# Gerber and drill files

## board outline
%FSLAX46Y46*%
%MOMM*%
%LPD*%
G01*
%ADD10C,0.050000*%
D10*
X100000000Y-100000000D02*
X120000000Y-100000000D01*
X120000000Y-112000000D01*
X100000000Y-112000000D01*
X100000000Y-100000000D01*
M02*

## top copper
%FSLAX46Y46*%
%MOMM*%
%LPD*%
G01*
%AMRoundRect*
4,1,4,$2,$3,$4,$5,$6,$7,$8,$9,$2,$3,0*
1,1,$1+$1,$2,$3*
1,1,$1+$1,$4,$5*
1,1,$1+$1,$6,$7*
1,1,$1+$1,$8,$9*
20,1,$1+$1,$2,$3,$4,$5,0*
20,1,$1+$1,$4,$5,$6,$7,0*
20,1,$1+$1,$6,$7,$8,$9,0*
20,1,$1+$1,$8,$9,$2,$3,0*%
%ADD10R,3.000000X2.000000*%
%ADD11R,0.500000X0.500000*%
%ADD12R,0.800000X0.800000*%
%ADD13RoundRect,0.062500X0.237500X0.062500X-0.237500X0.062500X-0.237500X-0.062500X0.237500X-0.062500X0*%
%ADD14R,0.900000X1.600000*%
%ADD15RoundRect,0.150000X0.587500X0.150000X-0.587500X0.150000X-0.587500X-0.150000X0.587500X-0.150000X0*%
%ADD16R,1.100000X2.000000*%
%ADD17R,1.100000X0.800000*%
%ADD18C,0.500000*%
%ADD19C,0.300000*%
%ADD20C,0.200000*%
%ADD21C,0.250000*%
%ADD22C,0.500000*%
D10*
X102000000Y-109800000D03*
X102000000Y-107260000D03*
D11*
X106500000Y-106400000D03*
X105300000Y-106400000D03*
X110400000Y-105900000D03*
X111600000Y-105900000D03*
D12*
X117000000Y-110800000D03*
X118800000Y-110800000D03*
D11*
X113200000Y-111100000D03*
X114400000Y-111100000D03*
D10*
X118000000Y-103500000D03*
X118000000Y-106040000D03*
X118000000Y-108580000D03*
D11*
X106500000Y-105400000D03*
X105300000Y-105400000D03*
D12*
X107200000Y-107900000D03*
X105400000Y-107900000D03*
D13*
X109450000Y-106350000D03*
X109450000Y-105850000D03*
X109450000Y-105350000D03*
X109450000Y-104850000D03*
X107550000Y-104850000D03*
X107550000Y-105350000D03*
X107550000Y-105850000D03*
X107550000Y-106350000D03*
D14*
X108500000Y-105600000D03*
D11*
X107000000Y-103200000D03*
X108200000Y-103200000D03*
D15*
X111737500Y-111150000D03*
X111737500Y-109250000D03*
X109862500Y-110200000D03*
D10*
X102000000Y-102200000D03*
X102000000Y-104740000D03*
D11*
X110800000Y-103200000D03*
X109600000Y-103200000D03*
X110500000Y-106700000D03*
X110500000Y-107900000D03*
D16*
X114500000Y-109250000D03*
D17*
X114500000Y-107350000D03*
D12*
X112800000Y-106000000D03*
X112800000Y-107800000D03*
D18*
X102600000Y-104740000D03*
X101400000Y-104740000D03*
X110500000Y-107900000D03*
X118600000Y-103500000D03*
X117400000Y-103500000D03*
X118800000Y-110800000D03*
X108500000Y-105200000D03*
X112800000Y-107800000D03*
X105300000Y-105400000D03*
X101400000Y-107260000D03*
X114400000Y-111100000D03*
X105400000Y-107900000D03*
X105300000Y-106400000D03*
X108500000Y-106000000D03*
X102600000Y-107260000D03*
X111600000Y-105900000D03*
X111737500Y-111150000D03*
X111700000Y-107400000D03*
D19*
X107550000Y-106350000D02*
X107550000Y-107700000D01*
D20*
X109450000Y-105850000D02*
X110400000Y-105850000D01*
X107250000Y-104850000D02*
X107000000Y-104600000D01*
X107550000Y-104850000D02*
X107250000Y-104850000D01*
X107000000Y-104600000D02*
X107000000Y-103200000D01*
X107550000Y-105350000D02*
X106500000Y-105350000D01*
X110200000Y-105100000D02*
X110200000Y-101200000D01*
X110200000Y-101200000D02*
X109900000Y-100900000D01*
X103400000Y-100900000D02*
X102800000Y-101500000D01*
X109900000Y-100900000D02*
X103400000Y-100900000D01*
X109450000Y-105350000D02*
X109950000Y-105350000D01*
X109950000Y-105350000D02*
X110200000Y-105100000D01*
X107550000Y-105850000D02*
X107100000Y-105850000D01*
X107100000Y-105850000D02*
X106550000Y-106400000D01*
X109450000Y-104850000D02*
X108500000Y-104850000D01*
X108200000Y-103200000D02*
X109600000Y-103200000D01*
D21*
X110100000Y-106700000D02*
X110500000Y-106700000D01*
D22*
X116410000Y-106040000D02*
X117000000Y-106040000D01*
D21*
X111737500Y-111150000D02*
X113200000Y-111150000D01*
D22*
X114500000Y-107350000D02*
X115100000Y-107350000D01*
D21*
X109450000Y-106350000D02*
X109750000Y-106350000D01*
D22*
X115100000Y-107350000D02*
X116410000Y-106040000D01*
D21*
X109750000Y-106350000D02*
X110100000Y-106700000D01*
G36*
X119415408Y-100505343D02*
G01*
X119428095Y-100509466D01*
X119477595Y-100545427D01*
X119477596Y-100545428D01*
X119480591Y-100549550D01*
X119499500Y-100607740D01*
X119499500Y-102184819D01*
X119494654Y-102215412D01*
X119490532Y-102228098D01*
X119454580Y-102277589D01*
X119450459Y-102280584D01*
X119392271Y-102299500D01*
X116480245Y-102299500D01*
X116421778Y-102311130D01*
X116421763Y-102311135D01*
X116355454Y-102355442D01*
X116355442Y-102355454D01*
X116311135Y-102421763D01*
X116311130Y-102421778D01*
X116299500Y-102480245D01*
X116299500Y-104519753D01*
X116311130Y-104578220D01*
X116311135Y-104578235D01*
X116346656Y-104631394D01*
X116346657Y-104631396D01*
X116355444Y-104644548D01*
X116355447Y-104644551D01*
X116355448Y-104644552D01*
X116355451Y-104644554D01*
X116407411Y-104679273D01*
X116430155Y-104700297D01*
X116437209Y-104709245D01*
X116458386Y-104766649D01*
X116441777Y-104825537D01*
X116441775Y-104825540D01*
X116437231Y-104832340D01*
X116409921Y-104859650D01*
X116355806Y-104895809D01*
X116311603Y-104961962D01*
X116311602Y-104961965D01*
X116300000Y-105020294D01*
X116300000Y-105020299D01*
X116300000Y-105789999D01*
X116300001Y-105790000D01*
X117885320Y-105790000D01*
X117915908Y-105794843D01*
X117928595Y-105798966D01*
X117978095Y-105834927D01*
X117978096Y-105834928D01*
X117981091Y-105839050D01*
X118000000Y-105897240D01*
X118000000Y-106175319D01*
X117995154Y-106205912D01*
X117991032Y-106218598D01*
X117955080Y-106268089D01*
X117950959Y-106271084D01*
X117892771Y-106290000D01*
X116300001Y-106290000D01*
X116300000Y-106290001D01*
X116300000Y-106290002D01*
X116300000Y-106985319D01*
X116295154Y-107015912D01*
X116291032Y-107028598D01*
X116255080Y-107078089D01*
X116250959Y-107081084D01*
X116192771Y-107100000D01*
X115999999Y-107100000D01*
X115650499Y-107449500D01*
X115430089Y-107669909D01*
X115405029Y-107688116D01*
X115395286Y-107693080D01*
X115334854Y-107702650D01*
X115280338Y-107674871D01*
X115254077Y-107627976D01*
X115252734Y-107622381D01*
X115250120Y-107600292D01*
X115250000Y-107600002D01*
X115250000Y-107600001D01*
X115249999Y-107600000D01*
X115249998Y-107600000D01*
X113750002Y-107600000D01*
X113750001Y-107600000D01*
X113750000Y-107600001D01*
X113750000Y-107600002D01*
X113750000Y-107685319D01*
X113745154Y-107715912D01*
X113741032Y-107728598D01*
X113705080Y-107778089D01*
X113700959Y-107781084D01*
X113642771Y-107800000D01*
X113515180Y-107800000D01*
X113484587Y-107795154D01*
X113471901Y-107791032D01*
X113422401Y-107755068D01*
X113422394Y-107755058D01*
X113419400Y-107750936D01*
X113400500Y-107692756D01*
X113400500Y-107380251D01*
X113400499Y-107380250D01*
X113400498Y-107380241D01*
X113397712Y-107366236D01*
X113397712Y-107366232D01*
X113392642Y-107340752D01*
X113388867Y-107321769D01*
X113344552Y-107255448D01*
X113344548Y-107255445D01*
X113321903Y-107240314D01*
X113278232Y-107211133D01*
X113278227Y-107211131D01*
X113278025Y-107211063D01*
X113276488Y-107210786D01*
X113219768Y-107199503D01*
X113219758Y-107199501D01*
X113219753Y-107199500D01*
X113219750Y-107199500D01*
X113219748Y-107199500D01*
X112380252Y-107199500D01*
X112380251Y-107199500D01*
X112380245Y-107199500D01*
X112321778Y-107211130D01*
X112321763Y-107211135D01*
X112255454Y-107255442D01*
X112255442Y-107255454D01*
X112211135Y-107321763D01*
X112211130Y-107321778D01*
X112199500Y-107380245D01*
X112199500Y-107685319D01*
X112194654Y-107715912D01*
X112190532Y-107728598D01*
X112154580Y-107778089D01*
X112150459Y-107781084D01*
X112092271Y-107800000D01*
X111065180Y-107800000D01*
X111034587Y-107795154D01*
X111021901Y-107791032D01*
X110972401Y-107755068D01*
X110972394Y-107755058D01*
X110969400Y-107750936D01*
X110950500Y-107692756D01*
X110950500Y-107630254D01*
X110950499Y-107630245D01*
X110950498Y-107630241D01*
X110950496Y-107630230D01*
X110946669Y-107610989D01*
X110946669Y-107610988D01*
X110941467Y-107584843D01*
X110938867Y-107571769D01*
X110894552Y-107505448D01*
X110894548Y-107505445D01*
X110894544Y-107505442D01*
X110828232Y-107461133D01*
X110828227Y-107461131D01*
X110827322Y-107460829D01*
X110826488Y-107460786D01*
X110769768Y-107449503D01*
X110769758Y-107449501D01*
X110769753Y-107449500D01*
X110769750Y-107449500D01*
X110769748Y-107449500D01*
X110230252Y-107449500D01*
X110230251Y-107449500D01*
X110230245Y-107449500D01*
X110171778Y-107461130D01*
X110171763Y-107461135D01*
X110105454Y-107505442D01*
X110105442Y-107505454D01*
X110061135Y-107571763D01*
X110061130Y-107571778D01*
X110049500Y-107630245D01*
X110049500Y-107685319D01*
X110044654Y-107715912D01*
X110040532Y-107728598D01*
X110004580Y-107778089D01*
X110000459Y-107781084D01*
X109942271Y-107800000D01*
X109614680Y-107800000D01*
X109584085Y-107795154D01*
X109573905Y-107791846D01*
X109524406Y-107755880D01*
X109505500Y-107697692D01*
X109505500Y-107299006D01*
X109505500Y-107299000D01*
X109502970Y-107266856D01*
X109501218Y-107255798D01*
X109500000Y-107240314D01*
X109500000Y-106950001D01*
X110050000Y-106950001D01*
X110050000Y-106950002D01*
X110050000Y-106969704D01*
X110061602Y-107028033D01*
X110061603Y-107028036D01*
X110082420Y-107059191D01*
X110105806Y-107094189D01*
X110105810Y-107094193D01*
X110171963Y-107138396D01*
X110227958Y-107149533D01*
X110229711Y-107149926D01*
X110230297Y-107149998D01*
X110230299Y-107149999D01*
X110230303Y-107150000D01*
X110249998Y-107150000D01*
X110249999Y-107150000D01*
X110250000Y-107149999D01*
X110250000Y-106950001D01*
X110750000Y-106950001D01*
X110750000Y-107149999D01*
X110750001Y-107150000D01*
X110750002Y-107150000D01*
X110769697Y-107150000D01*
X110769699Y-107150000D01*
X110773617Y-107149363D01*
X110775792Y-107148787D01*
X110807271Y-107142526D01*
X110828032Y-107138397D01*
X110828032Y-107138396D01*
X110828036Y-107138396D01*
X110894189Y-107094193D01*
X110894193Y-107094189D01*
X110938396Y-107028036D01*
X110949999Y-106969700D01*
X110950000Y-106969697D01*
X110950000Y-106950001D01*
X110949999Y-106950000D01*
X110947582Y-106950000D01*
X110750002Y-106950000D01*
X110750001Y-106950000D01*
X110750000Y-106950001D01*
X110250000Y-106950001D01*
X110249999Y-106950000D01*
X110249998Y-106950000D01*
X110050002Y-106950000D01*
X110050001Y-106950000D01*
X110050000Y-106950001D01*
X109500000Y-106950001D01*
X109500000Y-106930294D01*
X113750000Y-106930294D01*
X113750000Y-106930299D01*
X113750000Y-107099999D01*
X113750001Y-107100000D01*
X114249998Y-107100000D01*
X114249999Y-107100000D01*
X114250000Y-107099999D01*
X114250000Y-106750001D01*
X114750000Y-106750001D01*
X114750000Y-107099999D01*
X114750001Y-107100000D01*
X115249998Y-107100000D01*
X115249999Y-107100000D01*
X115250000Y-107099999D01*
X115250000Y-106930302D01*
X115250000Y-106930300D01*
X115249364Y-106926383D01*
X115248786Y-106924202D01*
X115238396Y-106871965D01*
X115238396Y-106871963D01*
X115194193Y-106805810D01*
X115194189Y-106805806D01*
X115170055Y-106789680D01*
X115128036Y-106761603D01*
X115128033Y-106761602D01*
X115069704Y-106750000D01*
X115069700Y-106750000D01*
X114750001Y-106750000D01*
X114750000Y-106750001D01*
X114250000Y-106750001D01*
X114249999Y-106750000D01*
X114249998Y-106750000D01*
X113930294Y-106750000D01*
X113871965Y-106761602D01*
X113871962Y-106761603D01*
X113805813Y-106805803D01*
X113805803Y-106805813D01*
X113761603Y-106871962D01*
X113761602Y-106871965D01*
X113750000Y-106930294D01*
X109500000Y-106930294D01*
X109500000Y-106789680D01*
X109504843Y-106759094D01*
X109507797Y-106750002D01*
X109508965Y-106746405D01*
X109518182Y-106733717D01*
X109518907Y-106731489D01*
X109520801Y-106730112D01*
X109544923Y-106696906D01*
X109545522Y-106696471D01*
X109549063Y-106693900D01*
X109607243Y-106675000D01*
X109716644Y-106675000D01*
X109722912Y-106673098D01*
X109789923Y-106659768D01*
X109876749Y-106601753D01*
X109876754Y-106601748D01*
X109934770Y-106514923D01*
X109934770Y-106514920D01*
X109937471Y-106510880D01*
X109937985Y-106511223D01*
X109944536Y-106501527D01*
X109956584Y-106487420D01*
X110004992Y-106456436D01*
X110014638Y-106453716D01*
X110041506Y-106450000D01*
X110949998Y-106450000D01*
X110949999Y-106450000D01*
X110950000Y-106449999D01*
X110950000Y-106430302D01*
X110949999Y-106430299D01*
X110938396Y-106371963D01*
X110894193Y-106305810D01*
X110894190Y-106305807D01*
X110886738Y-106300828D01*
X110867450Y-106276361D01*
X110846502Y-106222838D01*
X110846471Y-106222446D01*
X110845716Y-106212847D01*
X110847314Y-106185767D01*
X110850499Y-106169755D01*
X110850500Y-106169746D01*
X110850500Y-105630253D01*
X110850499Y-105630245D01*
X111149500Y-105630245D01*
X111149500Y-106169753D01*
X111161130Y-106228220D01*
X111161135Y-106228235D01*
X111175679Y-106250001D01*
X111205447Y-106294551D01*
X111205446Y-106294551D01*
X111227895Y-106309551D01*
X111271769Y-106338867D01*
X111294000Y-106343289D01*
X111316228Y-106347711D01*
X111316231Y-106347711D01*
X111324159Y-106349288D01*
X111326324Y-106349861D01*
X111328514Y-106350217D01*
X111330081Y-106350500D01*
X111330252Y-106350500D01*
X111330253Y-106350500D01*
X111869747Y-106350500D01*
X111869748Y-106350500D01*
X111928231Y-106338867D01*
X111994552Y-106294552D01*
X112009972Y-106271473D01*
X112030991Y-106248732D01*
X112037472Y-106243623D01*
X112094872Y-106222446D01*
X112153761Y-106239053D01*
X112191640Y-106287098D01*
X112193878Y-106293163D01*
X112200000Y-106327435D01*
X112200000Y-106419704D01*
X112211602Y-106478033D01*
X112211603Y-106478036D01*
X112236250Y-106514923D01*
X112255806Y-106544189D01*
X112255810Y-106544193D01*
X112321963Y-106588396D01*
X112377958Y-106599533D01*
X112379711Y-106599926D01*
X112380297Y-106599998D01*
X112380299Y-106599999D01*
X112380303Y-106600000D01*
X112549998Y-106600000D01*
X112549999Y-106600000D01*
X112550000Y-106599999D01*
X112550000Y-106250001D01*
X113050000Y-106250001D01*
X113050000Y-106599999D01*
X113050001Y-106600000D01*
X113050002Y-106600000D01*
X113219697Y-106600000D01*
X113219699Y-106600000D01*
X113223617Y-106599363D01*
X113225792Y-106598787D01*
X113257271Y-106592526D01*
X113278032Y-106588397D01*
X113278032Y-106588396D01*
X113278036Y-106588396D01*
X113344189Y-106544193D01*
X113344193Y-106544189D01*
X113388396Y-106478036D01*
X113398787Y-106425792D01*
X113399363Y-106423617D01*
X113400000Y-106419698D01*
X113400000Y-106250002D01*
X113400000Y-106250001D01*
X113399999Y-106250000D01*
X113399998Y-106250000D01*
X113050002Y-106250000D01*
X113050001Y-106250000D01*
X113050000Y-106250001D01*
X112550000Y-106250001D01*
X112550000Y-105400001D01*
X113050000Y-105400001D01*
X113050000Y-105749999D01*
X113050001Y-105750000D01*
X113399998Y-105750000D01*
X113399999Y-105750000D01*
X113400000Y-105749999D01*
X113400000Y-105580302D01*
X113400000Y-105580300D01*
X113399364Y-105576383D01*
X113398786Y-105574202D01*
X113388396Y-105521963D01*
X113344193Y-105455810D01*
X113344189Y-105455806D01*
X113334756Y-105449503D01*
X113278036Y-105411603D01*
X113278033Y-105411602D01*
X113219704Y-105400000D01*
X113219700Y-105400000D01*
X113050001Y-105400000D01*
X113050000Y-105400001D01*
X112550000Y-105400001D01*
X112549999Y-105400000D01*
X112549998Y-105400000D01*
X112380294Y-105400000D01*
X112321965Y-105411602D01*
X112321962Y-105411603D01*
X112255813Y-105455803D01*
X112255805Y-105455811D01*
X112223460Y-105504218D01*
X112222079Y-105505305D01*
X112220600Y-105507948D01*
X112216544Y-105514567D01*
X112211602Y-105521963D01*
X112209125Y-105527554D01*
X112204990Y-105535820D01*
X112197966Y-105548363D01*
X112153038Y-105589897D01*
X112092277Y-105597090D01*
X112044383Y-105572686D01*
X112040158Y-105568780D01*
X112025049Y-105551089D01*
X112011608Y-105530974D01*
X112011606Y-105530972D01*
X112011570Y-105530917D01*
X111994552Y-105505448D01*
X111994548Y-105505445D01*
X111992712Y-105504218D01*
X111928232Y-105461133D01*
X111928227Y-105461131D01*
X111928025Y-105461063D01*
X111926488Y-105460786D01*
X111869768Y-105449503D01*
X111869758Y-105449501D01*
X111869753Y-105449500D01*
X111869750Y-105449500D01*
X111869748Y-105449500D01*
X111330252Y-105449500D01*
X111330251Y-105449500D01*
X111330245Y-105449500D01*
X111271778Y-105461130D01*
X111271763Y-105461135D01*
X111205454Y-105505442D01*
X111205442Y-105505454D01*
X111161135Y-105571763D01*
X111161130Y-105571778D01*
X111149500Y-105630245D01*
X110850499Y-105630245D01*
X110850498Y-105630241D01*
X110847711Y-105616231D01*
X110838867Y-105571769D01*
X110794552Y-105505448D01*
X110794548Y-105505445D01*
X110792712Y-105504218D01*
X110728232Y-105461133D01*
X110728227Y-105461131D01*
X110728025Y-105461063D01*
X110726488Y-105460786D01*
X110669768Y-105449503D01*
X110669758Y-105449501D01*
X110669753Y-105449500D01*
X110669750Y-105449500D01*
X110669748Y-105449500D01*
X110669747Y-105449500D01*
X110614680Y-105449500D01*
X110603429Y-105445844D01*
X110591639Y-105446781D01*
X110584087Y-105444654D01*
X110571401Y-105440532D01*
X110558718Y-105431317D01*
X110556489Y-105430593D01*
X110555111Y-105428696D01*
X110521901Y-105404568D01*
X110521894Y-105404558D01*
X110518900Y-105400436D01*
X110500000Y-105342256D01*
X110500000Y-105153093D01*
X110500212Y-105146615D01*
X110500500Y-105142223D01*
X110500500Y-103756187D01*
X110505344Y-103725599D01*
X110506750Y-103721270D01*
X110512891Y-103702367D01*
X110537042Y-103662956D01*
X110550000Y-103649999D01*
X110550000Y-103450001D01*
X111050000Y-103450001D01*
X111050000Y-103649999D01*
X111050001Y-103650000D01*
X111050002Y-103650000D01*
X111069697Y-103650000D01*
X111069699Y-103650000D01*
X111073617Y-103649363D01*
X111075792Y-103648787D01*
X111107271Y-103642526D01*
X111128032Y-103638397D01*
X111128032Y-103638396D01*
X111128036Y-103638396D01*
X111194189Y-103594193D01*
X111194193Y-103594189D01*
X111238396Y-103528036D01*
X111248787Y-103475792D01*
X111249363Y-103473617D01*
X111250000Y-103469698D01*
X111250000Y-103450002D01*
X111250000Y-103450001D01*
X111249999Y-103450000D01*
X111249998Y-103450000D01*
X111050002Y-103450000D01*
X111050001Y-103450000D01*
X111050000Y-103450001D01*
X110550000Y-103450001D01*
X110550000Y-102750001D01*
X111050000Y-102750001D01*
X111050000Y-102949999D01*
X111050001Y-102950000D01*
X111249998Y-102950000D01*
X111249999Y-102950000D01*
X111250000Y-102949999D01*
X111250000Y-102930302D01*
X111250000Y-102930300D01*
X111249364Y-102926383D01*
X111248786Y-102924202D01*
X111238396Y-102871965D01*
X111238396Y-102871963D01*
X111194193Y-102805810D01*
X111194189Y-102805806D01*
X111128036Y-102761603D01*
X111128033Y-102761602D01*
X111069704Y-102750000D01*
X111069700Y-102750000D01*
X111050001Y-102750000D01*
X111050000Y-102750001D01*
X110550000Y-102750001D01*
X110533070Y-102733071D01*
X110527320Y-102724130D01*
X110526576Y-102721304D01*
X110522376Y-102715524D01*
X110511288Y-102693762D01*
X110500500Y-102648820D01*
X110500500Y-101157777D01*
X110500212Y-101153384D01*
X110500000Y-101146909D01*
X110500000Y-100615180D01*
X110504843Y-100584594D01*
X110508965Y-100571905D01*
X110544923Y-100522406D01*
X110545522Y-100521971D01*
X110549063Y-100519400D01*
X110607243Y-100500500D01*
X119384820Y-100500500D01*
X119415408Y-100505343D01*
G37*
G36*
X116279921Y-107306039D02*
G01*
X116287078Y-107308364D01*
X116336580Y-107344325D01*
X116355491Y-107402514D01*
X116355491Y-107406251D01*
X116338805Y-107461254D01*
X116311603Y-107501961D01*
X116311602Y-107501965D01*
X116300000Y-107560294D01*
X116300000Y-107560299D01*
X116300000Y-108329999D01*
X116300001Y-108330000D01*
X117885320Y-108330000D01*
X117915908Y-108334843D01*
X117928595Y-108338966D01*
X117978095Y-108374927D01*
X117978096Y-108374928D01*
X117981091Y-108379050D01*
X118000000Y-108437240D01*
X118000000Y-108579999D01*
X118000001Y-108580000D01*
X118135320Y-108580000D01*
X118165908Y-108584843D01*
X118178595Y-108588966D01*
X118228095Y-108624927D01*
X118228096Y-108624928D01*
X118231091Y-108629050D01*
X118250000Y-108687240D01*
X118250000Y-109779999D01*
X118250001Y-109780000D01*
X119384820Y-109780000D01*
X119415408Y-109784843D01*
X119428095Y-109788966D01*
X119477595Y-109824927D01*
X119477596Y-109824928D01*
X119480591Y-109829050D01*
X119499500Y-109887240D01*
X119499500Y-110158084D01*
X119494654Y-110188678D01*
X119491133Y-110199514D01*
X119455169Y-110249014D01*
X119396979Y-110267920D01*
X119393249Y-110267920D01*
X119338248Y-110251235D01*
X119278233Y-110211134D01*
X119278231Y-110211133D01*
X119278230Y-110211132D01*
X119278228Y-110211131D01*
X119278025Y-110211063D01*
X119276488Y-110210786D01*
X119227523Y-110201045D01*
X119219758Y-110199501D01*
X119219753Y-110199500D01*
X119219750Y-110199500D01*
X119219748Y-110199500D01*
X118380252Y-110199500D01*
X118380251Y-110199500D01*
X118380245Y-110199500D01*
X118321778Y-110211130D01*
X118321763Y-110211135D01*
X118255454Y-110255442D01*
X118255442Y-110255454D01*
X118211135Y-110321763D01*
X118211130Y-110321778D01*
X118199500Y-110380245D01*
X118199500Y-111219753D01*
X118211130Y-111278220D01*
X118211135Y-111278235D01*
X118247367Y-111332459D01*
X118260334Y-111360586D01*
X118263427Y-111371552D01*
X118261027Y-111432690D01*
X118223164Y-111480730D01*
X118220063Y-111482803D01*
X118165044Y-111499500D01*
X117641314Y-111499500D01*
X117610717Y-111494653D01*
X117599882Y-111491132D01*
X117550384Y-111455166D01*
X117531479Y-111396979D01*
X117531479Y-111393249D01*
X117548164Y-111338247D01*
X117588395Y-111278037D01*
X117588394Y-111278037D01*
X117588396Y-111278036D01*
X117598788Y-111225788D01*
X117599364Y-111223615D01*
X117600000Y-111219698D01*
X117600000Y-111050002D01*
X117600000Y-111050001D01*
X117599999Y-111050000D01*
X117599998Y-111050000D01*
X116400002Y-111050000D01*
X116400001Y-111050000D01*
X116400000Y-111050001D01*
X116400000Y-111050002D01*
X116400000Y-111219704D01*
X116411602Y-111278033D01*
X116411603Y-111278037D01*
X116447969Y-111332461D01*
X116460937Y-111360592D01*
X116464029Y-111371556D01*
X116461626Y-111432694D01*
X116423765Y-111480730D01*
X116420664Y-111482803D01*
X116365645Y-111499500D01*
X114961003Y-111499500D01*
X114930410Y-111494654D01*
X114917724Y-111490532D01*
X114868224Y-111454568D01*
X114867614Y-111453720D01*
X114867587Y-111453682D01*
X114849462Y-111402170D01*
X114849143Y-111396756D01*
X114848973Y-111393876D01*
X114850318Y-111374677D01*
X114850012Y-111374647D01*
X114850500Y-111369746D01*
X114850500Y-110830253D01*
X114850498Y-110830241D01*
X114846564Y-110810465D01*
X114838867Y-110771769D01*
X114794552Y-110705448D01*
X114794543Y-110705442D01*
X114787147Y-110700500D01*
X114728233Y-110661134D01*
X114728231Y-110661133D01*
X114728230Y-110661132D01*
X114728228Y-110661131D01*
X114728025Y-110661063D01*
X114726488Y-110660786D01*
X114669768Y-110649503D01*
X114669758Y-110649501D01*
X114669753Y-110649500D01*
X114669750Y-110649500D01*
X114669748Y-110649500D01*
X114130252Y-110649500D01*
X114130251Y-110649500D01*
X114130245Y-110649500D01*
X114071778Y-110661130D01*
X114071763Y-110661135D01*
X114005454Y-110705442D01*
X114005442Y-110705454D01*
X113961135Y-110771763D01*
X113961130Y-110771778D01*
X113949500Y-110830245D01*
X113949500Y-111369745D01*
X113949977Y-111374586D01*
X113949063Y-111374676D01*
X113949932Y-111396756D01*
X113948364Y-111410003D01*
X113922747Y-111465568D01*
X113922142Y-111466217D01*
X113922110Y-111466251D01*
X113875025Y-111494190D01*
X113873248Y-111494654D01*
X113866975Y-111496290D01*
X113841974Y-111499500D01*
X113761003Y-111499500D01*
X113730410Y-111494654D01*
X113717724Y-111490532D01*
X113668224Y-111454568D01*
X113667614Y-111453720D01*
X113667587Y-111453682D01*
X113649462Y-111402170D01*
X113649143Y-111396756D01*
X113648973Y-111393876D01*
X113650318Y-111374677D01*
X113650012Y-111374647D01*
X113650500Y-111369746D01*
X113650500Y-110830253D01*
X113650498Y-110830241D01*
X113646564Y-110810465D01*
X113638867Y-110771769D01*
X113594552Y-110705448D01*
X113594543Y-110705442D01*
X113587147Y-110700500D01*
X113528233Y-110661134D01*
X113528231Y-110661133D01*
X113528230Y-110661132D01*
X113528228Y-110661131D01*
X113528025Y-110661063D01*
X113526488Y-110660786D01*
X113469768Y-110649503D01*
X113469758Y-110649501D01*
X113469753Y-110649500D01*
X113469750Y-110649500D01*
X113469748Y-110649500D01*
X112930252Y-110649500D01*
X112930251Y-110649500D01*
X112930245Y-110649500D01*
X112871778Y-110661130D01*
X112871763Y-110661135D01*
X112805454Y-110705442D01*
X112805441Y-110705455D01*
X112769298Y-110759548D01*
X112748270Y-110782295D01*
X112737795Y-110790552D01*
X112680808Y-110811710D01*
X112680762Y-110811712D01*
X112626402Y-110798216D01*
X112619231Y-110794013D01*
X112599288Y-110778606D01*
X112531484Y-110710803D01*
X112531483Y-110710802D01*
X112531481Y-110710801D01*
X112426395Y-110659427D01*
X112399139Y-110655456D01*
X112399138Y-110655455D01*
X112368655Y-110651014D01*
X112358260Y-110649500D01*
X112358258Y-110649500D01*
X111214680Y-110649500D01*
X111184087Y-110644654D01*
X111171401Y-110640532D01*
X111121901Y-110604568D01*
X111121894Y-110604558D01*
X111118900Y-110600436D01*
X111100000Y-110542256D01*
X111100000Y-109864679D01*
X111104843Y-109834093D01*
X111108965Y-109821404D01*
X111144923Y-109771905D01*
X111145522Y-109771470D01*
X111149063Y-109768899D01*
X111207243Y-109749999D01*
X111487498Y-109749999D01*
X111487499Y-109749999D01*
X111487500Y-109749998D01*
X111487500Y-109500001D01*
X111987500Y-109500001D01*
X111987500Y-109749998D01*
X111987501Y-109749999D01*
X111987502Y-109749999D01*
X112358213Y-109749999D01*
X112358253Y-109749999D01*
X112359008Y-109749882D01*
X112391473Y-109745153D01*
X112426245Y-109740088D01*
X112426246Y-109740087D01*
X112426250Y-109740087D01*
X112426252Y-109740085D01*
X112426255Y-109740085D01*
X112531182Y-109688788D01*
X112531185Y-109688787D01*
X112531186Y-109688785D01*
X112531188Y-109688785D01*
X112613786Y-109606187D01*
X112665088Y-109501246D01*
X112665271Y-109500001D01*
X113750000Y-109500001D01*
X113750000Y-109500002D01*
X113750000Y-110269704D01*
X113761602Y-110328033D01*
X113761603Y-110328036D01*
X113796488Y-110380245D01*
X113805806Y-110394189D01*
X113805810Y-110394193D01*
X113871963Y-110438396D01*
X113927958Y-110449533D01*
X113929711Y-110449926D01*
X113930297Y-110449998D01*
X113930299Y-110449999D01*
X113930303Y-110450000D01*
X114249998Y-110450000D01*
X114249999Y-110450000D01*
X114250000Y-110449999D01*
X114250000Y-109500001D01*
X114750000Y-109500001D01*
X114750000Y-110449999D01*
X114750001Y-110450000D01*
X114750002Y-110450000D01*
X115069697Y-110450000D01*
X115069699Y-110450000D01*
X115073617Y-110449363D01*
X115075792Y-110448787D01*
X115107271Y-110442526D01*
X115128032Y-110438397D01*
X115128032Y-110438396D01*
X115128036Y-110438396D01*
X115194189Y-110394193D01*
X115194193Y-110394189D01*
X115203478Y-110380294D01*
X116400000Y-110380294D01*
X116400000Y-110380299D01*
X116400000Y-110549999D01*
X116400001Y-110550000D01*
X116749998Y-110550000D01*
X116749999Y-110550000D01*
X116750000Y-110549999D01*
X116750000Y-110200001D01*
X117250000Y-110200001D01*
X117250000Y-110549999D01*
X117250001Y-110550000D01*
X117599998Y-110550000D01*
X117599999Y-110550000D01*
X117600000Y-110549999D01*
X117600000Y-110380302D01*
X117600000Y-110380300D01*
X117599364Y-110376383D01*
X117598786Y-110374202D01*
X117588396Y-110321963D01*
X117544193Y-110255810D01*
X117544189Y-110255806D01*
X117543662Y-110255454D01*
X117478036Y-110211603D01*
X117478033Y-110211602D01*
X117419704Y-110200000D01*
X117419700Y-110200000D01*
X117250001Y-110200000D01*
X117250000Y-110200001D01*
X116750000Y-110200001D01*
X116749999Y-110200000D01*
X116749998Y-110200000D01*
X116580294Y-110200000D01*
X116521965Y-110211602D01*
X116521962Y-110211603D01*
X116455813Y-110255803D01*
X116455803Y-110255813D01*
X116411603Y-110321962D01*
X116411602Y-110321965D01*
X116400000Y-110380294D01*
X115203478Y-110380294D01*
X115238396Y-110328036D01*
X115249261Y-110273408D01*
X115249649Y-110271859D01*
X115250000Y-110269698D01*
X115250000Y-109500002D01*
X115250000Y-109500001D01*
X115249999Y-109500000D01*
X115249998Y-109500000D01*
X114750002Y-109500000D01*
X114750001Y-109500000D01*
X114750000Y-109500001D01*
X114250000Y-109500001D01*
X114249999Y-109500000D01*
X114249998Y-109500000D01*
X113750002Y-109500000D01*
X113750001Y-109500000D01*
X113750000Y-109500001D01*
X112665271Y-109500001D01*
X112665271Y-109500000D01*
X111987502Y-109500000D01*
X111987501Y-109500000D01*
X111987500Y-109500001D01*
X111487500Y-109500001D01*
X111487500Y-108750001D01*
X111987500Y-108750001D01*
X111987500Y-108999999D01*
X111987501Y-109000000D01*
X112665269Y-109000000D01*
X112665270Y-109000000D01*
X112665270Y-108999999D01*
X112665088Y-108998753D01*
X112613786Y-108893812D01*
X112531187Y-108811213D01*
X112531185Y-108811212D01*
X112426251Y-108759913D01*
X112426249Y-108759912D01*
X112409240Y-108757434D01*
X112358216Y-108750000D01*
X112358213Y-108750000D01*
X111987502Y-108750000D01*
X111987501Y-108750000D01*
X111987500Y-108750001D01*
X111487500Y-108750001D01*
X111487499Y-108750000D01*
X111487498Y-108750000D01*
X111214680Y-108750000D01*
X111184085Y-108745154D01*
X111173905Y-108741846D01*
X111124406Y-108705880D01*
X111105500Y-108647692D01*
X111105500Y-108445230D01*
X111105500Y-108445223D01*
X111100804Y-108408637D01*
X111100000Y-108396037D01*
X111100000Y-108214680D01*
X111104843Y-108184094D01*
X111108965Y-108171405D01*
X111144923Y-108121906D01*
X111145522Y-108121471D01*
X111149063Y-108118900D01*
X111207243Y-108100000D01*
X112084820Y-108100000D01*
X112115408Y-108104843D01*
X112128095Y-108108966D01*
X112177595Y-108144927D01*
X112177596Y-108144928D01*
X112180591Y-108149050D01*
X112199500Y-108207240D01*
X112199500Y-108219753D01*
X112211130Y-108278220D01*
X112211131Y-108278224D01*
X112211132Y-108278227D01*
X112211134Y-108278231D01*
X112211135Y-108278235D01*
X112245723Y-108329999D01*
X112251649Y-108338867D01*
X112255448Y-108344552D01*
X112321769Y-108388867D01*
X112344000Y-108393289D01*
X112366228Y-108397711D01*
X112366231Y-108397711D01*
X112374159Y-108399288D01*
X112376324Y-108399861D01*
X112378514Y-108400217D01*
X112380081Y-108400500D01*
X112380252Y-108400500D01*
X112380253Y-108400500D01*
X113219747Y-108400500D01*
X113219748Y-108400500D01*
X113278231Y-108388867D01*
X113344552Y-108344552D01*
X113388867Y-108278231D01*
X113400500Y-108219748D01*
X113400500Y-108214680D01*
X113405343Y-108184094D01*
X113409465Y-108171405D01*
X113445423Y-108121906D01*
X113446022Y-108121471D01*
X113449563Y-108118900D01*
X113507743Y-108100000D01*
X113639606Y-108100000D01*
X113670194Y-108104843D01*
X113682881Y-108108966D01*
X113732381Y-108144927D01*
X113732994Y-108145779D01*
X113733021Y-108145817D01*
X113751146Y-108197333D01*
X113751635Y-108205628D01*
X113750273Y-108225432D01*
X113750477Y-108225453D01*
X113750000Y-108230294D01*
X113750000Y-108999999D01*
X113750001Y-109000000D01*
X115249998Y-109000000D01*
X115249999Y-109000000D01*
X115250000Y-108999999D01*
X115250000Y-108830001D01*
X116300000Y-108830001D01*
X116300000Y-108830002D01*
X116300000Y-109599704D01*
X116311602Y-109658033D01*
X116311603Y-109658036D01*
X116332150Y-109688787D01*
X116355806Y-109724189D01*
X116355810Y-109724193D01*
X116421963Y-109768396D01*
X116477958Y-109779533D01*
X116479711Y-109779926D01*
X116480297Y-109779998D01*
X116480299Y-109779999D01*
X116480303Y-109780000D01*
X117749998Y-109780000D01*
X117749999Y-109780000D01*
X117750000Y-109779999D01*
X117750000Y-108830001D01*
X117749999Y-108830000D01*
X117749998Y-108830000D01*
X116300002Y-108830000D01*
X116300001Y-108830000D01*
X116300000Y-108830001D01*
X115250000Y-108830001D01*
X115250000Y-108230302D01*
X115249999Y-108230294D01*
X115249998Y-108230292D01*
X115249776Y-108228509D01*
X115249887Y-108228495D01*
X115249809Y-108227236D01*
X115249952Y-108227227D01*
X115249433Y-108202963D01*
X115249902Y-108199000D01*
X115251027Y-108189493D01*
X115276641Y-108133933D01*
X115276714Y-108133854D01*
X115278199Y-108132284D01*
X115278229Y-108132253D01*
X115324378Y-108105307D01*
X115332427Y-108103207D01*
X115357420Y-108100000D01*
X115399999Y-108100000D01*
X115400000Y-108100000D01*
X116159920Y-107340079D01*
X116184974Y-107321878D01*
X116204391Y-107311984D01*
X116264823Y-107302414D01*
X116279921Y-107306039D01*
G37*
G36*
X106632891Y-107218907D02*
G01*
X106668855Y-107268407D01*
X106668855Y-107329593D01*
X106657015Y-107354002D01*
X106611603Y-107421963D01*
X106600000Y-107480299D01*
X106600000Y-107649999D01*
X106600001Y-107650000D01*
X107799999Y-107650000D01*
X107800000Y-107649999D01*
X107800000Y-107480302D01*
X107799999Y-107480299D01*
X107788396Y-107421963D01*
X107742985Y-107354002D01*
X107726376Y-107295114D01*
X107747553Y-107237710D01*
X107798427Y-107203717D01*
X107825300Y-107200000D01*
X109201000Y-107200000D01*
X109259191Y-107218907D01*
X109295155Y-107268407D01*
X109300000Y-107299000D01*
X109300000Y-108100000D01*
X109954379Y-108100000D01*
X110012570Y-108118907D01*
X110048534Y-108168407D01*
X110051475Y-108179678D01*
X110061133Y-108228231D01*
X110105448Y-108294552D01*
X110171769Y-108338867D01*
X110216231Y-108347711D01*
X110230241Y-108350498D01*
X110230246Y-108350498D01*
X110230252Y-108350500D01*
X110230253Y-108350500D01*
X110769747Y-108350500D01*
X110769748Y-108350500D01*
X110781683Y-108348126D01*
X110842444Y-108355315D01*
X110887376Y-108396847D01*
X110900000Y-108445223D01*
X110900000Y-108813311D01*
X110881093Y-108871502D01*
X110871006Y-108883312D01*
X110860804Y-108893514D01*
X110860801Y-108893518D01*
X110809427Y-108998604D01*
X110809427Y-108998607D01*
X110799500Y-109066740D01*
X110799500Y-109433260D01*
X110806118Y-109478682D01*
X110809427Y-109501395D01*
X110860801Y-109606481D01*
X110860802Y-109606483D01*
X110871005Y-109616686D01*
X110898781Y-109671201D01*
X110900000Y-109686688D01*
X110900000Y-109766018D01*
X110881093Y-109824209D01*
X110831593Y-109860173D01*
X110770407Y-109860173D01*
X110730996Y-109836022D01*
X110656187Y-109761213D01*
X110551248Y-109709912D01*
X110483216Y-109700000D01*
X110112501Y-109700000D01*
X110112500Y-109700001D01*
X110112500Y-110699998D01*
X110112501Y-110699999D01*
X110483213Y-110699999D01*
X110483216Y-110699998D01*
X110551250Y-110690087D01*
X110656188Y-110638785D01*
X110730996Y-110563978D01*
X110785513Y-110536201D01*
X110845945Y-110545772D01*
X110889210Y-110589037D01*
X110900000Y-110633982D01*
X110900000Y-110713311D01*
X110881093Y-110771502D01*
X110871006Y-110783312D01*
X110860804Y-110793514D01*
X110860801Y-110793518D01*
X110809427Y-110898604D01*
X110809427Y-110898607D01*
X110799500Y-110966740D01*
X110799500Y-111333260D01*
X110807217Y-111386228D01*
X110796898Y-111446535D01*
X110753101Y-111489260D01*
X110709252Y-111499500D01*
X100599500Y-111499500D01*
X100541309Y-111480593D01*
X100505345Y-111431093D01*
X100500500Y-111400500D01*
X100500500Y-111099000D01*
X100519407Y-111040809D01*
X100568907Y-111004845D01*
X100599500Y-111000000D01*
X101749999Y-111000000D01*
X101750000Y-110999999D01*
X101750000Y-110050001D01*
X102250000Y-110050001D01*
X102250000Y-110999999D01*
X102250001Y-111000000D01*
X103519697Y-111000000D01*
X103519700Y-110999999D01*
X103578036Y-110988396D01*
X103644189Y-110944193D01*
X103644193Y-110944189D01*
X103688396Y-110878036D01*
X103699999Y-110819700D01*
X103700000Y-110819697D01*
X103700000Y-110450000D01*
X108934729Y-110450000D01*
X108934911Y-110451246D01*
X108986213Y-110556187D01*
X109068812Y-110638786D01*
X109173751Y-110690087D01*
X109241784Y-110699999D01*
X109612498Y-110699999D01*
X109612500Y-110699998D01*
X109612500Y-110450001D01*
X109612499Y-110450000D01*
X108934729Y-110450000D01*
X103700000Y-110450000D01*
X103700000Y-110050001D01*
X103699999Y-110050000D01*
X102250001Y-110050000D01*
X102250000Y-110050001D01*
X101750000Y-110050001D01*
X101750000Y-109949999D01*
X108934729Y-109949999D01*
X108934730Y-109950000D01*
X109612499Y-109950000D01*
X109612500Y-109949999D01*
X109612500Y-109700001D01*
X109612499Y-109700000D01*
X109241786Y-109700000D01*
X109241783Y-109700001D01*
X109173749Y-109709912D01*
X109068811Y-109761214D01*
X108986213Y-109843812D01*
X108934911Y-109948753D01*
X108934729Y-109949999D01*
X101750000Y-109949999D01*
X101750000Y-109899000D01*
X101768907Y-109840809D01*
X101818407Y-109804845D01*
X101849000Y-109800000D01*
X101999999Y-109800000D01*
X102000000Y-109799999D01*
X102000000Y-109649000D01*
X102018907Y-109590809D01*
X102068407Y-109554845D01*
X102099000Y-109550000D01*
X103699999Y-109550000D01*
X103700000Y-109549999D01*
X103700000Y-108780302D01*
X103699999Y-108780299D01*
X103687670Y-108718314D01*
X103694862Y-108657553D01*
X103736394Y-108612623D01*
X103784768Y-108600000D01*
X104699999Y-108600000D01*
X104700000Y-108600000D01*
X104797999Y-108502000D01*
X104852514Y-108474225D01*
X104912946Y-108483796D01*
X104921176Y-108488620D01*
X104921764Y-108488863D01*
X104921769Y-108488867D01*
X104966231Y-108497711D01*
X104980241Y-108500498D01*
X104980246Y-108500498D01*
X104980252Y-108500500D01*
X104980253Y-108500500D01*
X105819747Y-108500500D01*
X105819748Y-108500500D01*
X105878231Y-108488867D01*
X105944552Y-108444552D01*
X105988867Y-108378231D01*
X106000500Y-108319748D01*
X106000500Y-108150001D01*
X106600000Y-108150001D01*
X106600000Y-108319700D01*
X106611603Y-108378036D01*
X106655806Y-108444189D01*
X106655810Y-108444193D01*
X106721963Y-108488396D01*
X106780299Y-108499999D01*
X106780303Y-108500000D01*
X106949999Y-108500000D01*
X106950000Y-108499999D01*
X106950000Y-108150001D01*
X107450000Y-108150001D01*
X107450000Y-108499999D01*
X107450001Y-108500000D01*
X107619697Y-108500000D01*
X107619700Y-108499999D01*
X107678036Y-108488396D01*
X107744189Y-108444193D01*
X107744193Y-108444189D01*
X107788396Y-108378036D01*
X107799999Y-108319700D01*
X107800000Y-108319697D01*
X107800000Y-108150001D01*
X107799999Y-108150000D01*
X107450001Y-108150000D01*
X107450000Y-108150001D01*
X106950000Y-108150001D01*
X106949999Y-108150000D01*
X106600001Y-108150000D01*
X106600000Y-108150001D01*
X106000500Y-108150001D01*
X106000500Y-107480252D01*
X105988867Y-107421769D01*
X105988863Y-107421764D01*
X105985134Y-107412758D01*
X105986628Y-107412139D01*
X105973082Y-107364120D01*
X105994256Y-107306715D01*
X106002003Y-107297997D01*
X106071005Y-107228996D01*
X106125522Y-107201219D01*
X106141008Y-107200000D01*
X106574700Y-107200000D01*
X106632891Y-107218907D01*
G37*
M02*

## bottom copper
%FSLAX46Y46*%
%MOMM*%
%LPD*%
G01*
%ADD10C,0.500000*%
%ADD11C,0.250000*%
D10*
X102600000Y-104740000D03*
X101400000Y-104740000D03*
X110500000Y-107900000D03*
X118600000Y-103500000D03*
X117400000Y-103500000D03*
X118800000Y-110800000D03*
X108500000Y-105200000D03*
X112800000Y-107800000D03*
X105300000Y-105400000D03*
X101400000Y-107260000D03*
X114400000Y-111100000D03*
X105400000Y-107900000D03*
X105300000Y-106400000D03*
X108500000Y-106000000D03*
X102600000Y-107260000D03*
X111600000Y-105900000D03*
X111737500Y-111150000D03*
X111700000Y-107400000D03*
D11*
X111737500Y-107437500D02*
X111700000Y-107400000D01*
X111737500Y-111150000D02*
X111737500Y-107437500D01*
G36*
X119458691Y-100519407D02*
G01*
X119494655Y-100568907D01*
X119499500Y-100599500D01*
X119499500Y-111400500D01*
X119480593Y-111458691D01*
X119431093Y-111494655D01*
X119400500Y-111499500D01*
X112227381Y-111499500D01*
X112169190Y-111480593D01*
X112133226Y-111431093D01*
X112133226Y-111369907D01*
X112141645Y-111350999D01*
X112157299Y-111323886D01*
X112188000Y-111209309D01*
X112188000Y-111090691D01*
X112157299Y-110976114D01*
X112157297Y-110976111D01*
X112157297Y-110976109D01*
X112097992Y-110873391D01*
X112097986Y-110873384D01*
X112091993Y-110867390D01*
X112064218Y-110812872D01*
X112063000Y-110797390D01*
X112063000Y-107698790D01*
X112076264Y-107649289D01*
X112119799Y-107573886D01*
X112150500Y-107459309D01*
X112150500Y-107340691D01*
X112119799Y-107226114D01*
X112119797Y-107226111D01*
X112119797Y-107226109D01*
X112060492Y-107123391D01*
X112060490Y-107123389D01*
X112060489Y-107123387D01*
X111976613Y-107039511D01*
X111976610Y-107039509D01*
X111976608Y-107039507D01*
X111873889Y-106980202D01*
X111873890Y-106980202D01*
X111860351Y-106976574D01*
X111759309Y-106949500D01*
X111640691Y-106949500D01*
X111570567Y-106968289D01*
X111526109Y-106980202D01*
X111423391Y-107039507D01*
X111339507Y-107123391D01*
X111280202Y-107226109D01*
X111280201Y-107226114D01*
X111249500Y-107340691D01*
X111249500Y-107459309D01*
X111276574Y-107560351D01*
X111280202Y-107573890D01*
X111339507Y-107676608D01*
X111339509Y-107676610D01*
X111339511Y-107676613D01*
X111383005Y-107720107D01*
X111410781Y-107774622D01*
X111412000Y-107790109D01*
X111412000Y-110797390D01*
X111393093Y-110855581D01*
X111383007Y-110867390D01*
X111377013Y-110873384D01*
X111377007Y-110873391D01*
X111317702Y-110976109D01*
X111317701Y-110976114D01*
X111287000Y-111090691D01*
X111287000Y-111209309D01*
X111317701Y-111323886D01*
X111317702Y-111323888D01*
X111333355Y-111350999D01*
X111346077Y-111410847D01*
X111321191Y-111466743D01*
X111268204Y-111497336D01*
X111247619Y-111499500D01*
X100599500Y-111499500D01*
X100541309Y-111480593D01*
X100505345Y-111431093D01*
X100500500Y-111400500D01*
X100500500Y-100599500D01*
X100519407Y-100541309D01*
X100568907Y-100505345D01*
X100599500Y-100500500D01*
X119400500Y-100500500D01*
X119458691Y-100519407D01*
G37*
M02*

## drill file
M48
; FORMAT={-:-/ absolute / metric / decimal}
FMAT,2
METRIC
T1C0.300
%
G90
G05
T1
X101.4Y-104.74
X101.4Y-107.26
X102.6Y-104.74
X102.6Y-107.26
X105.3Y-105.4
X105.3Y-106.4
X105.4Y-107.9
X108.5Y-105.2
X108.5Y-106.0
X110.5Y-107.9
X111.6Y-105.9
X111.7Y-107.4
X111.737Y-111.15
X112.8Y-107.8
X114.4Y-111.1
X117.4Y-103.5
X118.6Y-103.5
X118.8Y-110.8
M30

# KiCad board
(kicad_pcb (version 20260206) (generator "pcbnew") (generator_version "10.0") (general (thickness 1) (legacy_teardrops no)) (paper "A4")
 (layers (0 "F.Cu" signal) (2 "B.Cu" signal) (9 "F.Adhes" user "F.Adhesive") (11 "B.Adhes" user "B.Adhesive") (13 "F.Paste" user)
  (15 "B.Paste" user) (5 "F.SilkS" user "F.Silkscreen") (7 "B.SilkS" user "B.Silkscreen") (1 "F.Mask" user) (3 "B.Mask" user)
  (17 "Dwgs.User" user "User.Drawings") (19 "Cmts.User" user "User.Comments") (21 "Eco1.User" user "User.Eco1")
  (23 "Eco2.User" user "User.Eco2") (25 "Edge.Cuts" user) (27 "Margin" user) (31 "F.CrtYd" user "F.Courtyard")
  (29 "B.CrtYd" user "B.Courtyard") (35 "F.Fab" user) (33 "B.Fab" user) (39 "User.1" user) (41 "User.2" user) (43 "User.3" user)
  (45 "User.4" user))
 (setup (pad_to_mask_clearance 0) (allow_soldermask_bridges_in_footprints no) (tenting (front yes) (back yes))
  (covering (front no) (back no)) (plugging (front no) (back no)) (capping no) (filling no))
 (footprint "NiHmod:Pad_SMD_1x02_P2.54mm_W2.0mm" (layer "F.Cu") (at 102 109.8 90)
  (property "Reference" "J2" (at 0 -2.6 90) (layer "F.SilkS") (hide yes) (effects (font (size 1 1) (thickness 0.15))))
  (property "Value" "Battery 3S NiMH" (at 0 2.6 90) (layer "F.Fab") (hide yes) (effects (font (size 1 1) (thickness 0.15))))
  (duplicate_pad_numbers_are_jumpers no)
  (pad "1" smd rect (at 0 0 90) (size 2 3) (layers "F.Cu" "F.Mask" "F.Paste") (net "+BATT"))
  (pad "2" smd rect (at 2.54 0 90) (size 2 3) (layers "F.Cu" "F.Mask" "F.Paste") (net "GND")))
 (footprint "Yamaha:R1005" (layer "F.Cu") (at 105.9 106.4 180)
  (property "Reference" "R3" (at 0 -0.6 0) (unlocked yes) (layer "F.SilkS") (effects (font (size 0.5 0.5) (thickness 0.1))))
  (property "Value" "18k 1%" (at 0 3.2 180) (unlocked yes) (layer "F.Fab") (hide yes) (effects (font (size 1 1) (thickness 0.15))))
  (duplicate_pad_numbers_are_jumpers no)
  (pad "1" smd rect (at -0.6 0) (size 0.5 0.5) (layers "F.Cu" "F.Mask" "F.Paste") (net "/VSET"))
  (pad "2" smd rect (at 0.6 0) (size 0.5 0.5) (layers "F.Cu" "F.Mask" "F.Paste") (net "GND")))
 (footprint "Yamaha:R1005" (layer "F.Cu") (at 111 105.9)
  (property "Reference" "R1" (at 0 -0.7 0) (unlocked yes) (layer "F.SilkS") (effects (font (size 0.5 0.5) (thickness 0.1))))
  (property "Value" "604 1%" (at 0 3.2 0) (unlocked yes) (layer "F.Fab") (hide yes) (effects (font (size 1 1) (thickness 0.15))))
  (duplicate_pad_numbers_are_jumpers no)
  (pad "1" smd rect (at -0.6 0 180) (size 0.5 0.5) (layers "F.Cu" "F.Mask" "F.Paste") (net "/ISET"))
  (pad "2" smd rect (at 0.6 0 180) (size 0.5 0.5) (layers "F.Cu" "F.Mask" "F.Paste") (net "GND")))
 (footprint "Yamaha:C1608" (layer "F.Cu") (at 117.9 110.8)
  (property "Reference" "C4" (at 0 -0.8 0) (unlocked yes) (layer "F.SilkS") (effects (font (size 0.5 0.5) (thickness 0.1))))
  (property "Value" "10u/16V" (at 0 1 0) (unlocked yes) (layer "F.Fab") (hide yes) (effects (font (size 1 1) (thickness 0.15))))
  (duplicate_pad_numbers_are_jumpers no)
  (pad "1" smd rect (at -0.9 0 180) (size 0.8 0.8) (layers "F.Cu" "F.Mask" "F.Paste") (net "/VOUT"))
  (pad "2" smd rect (at 0.9 0 180) (size 0.8 0.8) (layers "F.Cu" "F.Mask" "F.Paste") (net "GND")))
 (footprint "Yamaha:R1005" (layer "F.Cu") (at 113.8 111.1)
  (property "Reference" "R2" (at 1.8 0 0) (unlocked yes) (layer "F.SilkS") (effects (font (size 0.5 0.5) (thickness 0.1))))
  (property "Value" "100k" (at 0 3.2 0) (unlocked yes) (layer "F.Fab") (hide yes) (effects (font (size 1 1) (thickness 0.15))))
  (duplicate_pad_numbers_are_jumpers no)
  (pad "1" smd rect (at -0.6 0 180) (size 0.5 0.5) (layers "F.Cu" "F.Mask" "F.Paste") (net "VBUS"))
  (pad "2" smd rect (at 0.6 0 180) (size 0.5 0.5) (layers "F.Cu" "F.Mask" "F.Paste") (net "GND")))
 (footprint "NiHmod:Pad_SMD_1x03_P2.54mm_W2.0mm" (layer "F.Cu") (at 118 103.5 -90)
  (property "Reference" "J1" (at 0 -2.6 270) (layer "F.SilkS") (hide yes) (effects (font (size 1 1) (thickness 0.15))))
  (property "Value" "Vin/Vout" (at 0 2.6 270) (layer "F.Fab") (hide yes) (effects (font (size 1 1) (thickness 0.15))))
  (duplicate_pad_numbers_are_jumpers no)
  (pad "1" smd rect (at 0 0 270) (size 2 3) (layers "F.Cu" "F.Mask" "F.Paste") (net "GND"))
  (pad "2" smd rect (at 2.54 0 270) (size 2 3) (layers "F.Cu" "F.Mask" "F.Paste") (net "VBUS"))
  (pad "3" smd rect (at 5.08 0 270) (size 2 3) (layers "F.Cu" "F.Mask" "F.Paste") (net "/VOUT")))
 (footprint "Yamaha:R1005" (layer "F.Cu") (at 105.9 105.4 180)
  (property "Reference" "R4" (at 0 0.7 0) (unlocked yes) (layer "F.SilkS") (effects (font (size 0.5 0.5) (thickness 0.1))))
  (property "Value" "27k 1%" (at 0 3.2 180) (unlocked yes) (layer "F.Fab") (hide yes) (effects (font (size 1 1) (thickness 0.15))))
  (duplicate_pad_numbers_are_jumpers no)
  (pad "1" smd rect (at -0.6 0) (size 0.5 0.5) (layers "F.Cu" "F.Mask" "F.Paste") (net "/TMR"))
  (pad "2" smd rect (at 0.6 0) (size 0.5 0.5) (layers "F.Cu" "F.Mask" "F.Paste") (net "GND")))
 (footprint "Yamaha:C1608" (layer "F.Cu") (at 106.3 107.9 180)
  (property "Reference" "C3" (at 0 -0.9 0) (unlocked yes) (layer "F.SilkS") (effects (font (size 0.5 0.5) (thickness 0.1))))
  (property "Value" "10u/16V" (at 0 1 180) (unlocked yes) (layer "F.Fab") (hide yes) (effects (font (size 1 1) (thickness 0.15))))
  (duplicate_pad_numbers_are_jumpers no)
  (pad "1" smd rect (at -0.9 0) (size 0.8 0.8) (layers "F.Cu" "F.Mask" "F.Paste") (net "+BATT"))
  (pad "2" smd rect (at 0.9 0) (size 0.8 0.8) (layers "F.Cu" "F.Mask" "F.Paste") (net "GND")))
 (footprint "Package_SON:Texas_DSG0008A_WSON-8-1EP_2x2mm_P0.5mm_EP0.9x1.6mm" (layer "F.Cu") (at 108.5 105.6 180)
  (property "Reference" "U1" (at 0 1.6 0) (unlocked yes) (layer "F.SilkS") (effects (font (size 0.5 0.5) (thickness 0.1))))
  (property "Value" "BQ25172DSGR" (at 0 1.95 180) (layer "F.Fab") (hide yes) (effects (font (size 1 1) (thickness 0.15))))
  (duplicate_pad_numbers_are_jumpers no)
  (pad "" smd roundrect (at 0 -0.4 180) (size 0.73 0.64) (layers "F.Paste") (roundrect_rratio 0.25))
  (pad "" smd roundrect (at 0 0.4 180) (size 0.73 0.64) (layers "F.Paste") (roundrect_rratio 0.25))
  (pad "1" smd roundrect (at -0.95 -0.75 180) (size 0.6 0.25) (layers "F.Cu" "F.Mask" "F.Paste") (roundrect_rratio 0.25) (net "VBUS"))
  (pad "2" smd roundrect (at -0.95 -0.25 180) (size 0.6 0.25) (layers "F.Cu" "F.Mask" "F.Paste") (roundrect_rratio 0.25) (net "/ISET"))
  (pad "3" smd roundrect (at -0.95 0.25 180) (size 0.6 0.25) (layers "F.Cu" "F.Mask" "F.Paste") (roundrect_rratio 0.25) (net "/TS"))
  (pad "4" smd roundrect (at -0.95 0.75 180) (size 0.6 0.25) (layers "F.Cu" "F.Mask" "F.Paste") (roundrect_rratio 0.25) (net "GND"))
  (pad "5" smd roundrect (at 0.95 0.75 180) (size 0.6 0.25) (layers "F.Cu" "F.Mask" "F.Paste") (roundrect_rratio 0.25) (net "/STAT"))
  (pad "6" smd roundrect (at 0.95 0.25 180) (size 0.6 0.25) (layers "F.Cu" "F.Mask" "F.Paste") (roundrect_rratio 0.25) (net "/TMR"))
  (pad "7" smd roundrect (at 0.95 -0.25 180) (size 0.6 0.25) (layers "F.Cu" "F.Mask" "F.Paste") (roundrect_rratio 0.25) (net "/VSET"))
  (pad "8" smd roundrect (at 0.95 -0.75 180) (size 0.6 0.25) (layers "F.Cu" "F.Mask" "F.Paste") (roundrect_rratio 0.25) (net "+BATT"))
  (pad "9" smd rect (at 0 0 180) (size 0.9 1.6) (layers "F.Cu" "F.Mask") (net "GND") (zone_connect 2)))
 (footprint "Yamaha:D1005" (layer "F.Cu") (at 107.6 103.2)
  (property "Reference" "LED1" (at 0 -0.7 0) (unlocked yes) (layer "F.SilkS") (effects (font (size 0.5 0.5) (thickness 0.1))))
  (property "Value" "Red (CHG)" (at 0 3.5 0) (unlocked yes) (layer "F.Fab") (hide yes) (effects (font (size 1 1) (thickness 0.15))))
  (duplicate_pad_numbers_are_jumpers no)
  (pad "1" smd rect (at -0.6 0 180) (size 0.5 0.5) (layers "F.Cu" "F.Mask" "F.Paste") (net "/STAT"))
  (pad "2" smd rect (at 0.6 0 180) (size 0.5 0.5) (layers "F.Cu" "F.Mask" "F.Paste") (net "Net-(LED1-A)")))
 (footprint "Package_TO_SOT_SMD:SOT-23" (layer "F.Cu") (at 110.8 110.2 180)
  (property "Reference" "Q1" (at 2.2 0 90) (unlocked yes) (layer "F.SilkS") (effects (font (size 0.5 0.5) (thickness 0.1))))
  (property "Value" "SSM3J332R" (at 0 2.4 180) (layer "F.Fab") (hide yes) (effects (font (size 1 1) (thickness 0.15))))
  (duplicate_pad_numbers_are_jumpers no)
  (pad "1" smd roundrect (at -0.9375 -0.95 180) (size 1.475 0.6) (layers "F.Cu" "F.Mask" "F.Paste") (roundrect_rratio 0.25) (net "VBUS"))
  (pad "2" smd roundrect (at -0.9375 0.95 180) (size 1.475 0.6) (layers "F.Cu" "F.Mask" "F.Paste") (roundrect_rratio 0.25) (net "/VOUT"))
  (pad "3" smd roundrect (at 0.9375 0 180) (size 1.475 0.6) (layers "F.Cu" "F.Mask" "F.Paste") (roundrect_rratio 0.25) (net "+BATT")))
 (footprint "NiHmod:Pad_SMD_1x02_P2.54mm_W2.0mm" (layer "F.Cu") (at 102 102.2 -90)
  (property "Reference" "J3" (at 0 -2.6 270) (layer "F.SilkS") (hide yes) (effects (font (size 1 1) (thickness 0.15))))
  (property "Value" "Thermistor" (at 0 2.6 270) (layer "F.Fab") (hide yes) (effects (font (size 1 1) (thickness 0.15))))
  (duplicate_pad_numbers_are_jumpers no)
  (pad "1" smd rect (at 0 0 270) (size 2 3) (layers "F.Cu" "F.Mask" "F.Paste") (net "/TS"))
  (pad "2" smd rect (at 2.54 0 270) (size 2 3) (layers "F.Cu" "F.Mask" "F.Paste") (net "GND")))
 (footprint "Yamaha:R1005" (layer "F.Cu") (at 110.2 103.2 180)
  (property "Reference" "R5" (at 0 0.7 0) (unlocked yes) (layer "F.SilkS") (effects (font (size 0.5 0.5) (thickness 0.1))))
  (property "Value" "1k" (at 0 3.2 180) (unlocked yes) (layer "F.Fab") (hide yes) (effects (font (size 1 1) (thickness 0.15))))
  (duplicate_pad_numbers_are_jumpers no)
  (pad "1" smd rect (at -0.6 0) (size 0.5 0.5) (layers "F.Cu" "F.Mask" "F.Paste") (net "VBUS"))
  (pad "2" smd rect (at 0.6 0) (size 0.5 0.5) (layers "F.Cu" "F.Mask" "F.Paste") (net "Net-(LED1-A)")))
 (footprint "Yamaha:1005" (layer "F.Cu") (at 110.5 107.3 -90)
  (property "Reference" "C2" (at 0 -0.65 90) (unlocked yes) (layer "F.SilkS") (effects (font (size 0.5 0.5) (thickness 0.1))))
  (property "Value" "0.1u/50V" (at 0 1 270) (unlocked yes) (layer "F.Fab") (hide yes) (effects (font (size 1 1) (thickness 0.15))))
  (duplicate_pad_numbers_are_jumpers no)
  (pad "1" smd rect (at -0.6 0 90) (size 0.5 0.5) (layers "F.Cu" "F.Mask" "F.Paste") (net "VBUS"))
  (pad "2" smd rect (at 0.6 0 90) (size 0.5 0.5) (layers "F.Cu" "F.Mask" "F.Paste") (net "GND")))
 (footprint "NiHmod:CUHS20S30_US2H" (layer "F.Cu") (at 114.5 108.6 90)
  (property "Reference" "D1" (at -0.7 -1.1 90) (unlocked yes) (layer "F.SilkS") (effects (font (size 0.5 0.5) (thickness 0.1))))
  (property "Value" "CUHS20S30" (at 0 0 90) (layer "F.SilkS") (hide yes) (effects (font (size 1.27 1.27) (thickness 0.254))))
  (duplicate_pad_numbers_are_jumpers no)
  (pad "1" smd rect (at -0.65 0 180) (size 1.1 2) (layers "F.Cu" "F.Mask" "F.Paste") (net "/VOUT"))
  (pad "2" smd rect (at 1.25 0 90) (size 0.8 1.1) (layers "F.Cu" "F.Mask" "F.Paste") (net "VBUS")))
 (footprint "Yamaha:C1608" (layer "F.Cu") (at 112.8 106.9 -90)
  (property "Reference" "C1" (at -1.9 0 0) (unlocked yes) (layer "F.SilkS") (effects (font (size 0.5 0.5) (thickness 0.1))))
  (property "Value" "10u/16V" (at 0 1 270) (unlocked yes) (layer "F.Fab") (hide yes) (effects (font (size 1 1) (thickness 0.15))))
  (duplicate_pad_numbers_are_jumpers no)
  (pad "1" smd rect (at -0.9 0 90) (size 0.8 0.8) (layers "F.Cu" "F.Mask" "F.Paste") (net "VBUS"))
  (pad "2" smd rect (at 0.9 0 90) (size 0.8 0.8) (layers "F.Cu" "F.Mask" "F.Paste") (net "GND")))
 (gr_rect (start 100 100) (end 120 112) (stroke (width 0.05) (type default)) (fill no) (layer "Edge.Cuts"))
 (segment (start 107.55 106.35) (end 107.55 107.7) (width 0.3) (layer "F.Cu") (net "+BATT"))
 (segment (start 109.45 105.85) (end 110.4 105.85) (width 0.2) (layer "F.Cu") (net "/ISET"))
 (segment (start 107.25 104.85) (end 107 104.6) (width 0.2) (layer "F.Cu") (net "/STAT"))
 (segment (start 107.55 104.85) (end 107.25 104.85) (width 0.2) (layer "F.Cu") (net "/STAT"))
 (segment (start 107 104.6) (end 107 103.2) (width 0.2) (layer "F.Cu") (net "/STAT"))
 (segment (start 107.55 105.35) (end 106.5 105.35) (width 0.2) (layer "F.Cu") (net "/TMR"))
 (segment (start 110.2 105.1) (end 110.2 101.2) (width 0.2) (layer "F.Cu") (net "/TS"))
 (segment (start 110.2 101.2) (end 109.9 100.9) (width 0.2) (layer "F.Cu") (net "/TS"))
 (segment (start 103.4 100.9) (end 102.8 101.5) (width 0.2) (layer "F.Cu") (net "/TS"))
 (segment (start 109.9 100.9) (end 103.4 100.9) (width 0.2) (layer "F.Cu") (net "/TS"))
 (segment (start 109.45 105.35) (end 109.95 105.35) (width 0.2) (layer "F.Cu") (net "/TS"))
 (segment (start 109.95 105.35) (end 110.2 105.1) (width 0.2) (layer "F.Cu") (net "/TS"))
 (segment (start 107.55 105.85) (end 107.1 105.85) (width 0.2) (layer "F.Cu") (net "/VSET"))
 (segment (start 107.1 105.85) (end 106.55 106.4) (width 0.2) (layer "F.Cu") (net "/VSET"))
 (segment (start 109.45 104.85) (end 108.5 104.85) (width 0.2) (layer "F.Cu") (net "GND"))
 (via (at 102.6 104.74) (size 0.5) (drill 0.3) (layers "F.Cu" "B.Cu") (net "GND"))
 (via (at 101.4 104.74) (size 0.5) (drill 0.3) (layers "F.Cu" "B.Cu") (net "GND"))
 (via (at 110.5 107.9) (size 0.5) (drill 0.3) (layers "F.Cu" "B.Cu") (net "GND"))
 (via (at 118.6 103.5) (size 0.5) (drill 0.3) (layers "F.Cu" "B.Cu") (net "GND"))
 (via (at 117.4 103.5) (size 0.5) (drill 0.3) (layers "F.Cu" "B.Cu") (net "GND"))
 (via (at 118.8 110.8) (size 0.5) (drill 0.3) (layers "F.Cu" "B.Cu") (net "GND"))
 (via (at 108.5 105.2) (size 0.5) (drill 0.3) (layers "F.Cu" "B.Cu") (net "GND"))
 (via (at 112.8 107.8) (size 0.5) (drill 0.3) (layers "F.Cu" "B.Cu") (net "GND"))
 (via (at 105.3 105.4) (size 0.5) (drill 0.3) (layers "F.Cu" "B.Cu") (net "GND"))
 (via (at 101.4 107.26) (size 0.5) (drill 0.3) (layers "F.Cu" "B.Cu") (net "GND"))
 (via (at 114.4 111.1) (size 0.5) (drill 0.3) (layers "F.Cu" "B.Cu") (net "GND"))
 (via (at 105.4 107.9) (size 0.5) (drill 0.3) (layers "F.Cu" "B.Cu") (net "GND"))
 (via (at 105.3 106.4) (size 0.5) (drill 0.3) (layers "F.Cu" "B.Cu") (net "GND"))
 (via (at 108.5 106) (size 0.5) (drill 0.3) (layers "F.Cu" "B.Cu") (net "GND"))
 (via (at 102.6 107.26) (size 0.5) (drill 0.3) (layers "F.Cu" "B.Cu") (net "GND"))
 (via (at 111.6 105.9) (size 0.5) (drill 0.3) (layers "F.Cu" "B.Cu") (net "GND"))
 (segment (start 108.2 103.2) (end 109.6 103.2) (width 0.2) (layer "F.Cu") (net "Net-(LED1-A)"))
 (segment (start 110.1 106.7) (end 110.5 106.7) (width 0.25) (layer "F.Cu") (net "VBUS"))
 (segment (start 116.41 106.04) (end 117 106.04) (width 0.5) (layer "F.Cu") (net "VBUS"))
 (segment (start 111.7375 111.15) (end 113.2 111.15) (width 0.25) (layer "F.Cu") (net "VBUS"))
 (segment (start 114.5 107.35) (end 115.1 107.35) (width 0.5) (layer "F.Cu") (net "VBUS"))
 (segment (start 109.45 106.35) (end 109.75 106.35) (width 0.25) (layer "F.Cu") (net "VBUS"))
 (segment (start 115.1 107.35) (end 116.41 106.04) (width 0.5) (layer "F.Cu") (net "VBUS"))
 (segment (start 109.75 106.35) (end 110.1 106.7) (width 0.25) (layer "F.Cu") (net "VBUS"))
 (via (at 111.7375 111.15) (size 0.5) (drill 0.3) (layers "F.Cu" "B.Cu") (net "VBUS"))
 (via (at 111.7 107.4) (size 0.5) (drill 0.3) (layers "F.Cu" "B.Cu") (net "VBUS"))
 (segment (start 111.7375 107.4375) (end 111.7 107.4) (width 0.25) (layer "B.Cu") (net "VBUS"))
 (segment (start 111.7375 111.15) (end 111.7375 107.4375) (width 0.25) (layer "B.Cu") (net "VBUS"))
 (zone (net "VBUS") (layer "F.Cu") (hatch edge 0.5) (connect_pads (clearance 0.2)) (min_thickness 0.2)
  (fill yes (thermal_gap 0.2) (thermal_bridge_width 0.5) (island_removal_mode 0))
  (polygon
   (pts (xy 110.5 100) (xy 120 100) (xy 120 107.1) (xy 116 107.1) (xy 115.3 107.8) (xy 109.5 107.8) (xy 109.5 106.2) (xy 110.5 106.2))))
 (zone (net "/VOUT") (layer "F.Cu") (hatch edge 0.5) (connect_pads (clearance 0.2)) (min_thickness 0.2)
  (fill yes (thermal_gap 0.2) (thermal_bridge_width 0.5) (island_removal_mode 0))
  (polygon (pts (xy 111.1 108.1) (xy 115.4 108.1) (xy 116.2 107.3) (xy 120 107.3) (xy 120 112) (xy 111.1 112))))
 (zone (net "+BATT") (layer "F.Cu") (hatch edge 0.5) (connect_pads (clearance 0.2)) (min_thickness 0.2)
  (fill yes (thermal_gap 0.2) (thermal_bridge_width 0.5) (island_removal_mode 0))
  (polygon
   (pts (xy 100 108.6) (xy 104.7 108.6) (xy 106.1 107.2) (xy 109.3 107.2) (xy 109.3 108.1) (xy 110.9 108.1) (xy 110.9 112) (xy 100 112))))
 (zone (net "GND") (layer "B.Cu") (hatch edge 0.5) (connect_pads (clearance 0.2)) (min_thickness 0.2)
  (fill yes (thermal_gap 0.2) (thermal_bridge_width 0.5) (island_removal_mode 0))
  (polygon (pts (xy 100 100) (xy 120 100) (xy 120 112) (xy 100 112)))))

